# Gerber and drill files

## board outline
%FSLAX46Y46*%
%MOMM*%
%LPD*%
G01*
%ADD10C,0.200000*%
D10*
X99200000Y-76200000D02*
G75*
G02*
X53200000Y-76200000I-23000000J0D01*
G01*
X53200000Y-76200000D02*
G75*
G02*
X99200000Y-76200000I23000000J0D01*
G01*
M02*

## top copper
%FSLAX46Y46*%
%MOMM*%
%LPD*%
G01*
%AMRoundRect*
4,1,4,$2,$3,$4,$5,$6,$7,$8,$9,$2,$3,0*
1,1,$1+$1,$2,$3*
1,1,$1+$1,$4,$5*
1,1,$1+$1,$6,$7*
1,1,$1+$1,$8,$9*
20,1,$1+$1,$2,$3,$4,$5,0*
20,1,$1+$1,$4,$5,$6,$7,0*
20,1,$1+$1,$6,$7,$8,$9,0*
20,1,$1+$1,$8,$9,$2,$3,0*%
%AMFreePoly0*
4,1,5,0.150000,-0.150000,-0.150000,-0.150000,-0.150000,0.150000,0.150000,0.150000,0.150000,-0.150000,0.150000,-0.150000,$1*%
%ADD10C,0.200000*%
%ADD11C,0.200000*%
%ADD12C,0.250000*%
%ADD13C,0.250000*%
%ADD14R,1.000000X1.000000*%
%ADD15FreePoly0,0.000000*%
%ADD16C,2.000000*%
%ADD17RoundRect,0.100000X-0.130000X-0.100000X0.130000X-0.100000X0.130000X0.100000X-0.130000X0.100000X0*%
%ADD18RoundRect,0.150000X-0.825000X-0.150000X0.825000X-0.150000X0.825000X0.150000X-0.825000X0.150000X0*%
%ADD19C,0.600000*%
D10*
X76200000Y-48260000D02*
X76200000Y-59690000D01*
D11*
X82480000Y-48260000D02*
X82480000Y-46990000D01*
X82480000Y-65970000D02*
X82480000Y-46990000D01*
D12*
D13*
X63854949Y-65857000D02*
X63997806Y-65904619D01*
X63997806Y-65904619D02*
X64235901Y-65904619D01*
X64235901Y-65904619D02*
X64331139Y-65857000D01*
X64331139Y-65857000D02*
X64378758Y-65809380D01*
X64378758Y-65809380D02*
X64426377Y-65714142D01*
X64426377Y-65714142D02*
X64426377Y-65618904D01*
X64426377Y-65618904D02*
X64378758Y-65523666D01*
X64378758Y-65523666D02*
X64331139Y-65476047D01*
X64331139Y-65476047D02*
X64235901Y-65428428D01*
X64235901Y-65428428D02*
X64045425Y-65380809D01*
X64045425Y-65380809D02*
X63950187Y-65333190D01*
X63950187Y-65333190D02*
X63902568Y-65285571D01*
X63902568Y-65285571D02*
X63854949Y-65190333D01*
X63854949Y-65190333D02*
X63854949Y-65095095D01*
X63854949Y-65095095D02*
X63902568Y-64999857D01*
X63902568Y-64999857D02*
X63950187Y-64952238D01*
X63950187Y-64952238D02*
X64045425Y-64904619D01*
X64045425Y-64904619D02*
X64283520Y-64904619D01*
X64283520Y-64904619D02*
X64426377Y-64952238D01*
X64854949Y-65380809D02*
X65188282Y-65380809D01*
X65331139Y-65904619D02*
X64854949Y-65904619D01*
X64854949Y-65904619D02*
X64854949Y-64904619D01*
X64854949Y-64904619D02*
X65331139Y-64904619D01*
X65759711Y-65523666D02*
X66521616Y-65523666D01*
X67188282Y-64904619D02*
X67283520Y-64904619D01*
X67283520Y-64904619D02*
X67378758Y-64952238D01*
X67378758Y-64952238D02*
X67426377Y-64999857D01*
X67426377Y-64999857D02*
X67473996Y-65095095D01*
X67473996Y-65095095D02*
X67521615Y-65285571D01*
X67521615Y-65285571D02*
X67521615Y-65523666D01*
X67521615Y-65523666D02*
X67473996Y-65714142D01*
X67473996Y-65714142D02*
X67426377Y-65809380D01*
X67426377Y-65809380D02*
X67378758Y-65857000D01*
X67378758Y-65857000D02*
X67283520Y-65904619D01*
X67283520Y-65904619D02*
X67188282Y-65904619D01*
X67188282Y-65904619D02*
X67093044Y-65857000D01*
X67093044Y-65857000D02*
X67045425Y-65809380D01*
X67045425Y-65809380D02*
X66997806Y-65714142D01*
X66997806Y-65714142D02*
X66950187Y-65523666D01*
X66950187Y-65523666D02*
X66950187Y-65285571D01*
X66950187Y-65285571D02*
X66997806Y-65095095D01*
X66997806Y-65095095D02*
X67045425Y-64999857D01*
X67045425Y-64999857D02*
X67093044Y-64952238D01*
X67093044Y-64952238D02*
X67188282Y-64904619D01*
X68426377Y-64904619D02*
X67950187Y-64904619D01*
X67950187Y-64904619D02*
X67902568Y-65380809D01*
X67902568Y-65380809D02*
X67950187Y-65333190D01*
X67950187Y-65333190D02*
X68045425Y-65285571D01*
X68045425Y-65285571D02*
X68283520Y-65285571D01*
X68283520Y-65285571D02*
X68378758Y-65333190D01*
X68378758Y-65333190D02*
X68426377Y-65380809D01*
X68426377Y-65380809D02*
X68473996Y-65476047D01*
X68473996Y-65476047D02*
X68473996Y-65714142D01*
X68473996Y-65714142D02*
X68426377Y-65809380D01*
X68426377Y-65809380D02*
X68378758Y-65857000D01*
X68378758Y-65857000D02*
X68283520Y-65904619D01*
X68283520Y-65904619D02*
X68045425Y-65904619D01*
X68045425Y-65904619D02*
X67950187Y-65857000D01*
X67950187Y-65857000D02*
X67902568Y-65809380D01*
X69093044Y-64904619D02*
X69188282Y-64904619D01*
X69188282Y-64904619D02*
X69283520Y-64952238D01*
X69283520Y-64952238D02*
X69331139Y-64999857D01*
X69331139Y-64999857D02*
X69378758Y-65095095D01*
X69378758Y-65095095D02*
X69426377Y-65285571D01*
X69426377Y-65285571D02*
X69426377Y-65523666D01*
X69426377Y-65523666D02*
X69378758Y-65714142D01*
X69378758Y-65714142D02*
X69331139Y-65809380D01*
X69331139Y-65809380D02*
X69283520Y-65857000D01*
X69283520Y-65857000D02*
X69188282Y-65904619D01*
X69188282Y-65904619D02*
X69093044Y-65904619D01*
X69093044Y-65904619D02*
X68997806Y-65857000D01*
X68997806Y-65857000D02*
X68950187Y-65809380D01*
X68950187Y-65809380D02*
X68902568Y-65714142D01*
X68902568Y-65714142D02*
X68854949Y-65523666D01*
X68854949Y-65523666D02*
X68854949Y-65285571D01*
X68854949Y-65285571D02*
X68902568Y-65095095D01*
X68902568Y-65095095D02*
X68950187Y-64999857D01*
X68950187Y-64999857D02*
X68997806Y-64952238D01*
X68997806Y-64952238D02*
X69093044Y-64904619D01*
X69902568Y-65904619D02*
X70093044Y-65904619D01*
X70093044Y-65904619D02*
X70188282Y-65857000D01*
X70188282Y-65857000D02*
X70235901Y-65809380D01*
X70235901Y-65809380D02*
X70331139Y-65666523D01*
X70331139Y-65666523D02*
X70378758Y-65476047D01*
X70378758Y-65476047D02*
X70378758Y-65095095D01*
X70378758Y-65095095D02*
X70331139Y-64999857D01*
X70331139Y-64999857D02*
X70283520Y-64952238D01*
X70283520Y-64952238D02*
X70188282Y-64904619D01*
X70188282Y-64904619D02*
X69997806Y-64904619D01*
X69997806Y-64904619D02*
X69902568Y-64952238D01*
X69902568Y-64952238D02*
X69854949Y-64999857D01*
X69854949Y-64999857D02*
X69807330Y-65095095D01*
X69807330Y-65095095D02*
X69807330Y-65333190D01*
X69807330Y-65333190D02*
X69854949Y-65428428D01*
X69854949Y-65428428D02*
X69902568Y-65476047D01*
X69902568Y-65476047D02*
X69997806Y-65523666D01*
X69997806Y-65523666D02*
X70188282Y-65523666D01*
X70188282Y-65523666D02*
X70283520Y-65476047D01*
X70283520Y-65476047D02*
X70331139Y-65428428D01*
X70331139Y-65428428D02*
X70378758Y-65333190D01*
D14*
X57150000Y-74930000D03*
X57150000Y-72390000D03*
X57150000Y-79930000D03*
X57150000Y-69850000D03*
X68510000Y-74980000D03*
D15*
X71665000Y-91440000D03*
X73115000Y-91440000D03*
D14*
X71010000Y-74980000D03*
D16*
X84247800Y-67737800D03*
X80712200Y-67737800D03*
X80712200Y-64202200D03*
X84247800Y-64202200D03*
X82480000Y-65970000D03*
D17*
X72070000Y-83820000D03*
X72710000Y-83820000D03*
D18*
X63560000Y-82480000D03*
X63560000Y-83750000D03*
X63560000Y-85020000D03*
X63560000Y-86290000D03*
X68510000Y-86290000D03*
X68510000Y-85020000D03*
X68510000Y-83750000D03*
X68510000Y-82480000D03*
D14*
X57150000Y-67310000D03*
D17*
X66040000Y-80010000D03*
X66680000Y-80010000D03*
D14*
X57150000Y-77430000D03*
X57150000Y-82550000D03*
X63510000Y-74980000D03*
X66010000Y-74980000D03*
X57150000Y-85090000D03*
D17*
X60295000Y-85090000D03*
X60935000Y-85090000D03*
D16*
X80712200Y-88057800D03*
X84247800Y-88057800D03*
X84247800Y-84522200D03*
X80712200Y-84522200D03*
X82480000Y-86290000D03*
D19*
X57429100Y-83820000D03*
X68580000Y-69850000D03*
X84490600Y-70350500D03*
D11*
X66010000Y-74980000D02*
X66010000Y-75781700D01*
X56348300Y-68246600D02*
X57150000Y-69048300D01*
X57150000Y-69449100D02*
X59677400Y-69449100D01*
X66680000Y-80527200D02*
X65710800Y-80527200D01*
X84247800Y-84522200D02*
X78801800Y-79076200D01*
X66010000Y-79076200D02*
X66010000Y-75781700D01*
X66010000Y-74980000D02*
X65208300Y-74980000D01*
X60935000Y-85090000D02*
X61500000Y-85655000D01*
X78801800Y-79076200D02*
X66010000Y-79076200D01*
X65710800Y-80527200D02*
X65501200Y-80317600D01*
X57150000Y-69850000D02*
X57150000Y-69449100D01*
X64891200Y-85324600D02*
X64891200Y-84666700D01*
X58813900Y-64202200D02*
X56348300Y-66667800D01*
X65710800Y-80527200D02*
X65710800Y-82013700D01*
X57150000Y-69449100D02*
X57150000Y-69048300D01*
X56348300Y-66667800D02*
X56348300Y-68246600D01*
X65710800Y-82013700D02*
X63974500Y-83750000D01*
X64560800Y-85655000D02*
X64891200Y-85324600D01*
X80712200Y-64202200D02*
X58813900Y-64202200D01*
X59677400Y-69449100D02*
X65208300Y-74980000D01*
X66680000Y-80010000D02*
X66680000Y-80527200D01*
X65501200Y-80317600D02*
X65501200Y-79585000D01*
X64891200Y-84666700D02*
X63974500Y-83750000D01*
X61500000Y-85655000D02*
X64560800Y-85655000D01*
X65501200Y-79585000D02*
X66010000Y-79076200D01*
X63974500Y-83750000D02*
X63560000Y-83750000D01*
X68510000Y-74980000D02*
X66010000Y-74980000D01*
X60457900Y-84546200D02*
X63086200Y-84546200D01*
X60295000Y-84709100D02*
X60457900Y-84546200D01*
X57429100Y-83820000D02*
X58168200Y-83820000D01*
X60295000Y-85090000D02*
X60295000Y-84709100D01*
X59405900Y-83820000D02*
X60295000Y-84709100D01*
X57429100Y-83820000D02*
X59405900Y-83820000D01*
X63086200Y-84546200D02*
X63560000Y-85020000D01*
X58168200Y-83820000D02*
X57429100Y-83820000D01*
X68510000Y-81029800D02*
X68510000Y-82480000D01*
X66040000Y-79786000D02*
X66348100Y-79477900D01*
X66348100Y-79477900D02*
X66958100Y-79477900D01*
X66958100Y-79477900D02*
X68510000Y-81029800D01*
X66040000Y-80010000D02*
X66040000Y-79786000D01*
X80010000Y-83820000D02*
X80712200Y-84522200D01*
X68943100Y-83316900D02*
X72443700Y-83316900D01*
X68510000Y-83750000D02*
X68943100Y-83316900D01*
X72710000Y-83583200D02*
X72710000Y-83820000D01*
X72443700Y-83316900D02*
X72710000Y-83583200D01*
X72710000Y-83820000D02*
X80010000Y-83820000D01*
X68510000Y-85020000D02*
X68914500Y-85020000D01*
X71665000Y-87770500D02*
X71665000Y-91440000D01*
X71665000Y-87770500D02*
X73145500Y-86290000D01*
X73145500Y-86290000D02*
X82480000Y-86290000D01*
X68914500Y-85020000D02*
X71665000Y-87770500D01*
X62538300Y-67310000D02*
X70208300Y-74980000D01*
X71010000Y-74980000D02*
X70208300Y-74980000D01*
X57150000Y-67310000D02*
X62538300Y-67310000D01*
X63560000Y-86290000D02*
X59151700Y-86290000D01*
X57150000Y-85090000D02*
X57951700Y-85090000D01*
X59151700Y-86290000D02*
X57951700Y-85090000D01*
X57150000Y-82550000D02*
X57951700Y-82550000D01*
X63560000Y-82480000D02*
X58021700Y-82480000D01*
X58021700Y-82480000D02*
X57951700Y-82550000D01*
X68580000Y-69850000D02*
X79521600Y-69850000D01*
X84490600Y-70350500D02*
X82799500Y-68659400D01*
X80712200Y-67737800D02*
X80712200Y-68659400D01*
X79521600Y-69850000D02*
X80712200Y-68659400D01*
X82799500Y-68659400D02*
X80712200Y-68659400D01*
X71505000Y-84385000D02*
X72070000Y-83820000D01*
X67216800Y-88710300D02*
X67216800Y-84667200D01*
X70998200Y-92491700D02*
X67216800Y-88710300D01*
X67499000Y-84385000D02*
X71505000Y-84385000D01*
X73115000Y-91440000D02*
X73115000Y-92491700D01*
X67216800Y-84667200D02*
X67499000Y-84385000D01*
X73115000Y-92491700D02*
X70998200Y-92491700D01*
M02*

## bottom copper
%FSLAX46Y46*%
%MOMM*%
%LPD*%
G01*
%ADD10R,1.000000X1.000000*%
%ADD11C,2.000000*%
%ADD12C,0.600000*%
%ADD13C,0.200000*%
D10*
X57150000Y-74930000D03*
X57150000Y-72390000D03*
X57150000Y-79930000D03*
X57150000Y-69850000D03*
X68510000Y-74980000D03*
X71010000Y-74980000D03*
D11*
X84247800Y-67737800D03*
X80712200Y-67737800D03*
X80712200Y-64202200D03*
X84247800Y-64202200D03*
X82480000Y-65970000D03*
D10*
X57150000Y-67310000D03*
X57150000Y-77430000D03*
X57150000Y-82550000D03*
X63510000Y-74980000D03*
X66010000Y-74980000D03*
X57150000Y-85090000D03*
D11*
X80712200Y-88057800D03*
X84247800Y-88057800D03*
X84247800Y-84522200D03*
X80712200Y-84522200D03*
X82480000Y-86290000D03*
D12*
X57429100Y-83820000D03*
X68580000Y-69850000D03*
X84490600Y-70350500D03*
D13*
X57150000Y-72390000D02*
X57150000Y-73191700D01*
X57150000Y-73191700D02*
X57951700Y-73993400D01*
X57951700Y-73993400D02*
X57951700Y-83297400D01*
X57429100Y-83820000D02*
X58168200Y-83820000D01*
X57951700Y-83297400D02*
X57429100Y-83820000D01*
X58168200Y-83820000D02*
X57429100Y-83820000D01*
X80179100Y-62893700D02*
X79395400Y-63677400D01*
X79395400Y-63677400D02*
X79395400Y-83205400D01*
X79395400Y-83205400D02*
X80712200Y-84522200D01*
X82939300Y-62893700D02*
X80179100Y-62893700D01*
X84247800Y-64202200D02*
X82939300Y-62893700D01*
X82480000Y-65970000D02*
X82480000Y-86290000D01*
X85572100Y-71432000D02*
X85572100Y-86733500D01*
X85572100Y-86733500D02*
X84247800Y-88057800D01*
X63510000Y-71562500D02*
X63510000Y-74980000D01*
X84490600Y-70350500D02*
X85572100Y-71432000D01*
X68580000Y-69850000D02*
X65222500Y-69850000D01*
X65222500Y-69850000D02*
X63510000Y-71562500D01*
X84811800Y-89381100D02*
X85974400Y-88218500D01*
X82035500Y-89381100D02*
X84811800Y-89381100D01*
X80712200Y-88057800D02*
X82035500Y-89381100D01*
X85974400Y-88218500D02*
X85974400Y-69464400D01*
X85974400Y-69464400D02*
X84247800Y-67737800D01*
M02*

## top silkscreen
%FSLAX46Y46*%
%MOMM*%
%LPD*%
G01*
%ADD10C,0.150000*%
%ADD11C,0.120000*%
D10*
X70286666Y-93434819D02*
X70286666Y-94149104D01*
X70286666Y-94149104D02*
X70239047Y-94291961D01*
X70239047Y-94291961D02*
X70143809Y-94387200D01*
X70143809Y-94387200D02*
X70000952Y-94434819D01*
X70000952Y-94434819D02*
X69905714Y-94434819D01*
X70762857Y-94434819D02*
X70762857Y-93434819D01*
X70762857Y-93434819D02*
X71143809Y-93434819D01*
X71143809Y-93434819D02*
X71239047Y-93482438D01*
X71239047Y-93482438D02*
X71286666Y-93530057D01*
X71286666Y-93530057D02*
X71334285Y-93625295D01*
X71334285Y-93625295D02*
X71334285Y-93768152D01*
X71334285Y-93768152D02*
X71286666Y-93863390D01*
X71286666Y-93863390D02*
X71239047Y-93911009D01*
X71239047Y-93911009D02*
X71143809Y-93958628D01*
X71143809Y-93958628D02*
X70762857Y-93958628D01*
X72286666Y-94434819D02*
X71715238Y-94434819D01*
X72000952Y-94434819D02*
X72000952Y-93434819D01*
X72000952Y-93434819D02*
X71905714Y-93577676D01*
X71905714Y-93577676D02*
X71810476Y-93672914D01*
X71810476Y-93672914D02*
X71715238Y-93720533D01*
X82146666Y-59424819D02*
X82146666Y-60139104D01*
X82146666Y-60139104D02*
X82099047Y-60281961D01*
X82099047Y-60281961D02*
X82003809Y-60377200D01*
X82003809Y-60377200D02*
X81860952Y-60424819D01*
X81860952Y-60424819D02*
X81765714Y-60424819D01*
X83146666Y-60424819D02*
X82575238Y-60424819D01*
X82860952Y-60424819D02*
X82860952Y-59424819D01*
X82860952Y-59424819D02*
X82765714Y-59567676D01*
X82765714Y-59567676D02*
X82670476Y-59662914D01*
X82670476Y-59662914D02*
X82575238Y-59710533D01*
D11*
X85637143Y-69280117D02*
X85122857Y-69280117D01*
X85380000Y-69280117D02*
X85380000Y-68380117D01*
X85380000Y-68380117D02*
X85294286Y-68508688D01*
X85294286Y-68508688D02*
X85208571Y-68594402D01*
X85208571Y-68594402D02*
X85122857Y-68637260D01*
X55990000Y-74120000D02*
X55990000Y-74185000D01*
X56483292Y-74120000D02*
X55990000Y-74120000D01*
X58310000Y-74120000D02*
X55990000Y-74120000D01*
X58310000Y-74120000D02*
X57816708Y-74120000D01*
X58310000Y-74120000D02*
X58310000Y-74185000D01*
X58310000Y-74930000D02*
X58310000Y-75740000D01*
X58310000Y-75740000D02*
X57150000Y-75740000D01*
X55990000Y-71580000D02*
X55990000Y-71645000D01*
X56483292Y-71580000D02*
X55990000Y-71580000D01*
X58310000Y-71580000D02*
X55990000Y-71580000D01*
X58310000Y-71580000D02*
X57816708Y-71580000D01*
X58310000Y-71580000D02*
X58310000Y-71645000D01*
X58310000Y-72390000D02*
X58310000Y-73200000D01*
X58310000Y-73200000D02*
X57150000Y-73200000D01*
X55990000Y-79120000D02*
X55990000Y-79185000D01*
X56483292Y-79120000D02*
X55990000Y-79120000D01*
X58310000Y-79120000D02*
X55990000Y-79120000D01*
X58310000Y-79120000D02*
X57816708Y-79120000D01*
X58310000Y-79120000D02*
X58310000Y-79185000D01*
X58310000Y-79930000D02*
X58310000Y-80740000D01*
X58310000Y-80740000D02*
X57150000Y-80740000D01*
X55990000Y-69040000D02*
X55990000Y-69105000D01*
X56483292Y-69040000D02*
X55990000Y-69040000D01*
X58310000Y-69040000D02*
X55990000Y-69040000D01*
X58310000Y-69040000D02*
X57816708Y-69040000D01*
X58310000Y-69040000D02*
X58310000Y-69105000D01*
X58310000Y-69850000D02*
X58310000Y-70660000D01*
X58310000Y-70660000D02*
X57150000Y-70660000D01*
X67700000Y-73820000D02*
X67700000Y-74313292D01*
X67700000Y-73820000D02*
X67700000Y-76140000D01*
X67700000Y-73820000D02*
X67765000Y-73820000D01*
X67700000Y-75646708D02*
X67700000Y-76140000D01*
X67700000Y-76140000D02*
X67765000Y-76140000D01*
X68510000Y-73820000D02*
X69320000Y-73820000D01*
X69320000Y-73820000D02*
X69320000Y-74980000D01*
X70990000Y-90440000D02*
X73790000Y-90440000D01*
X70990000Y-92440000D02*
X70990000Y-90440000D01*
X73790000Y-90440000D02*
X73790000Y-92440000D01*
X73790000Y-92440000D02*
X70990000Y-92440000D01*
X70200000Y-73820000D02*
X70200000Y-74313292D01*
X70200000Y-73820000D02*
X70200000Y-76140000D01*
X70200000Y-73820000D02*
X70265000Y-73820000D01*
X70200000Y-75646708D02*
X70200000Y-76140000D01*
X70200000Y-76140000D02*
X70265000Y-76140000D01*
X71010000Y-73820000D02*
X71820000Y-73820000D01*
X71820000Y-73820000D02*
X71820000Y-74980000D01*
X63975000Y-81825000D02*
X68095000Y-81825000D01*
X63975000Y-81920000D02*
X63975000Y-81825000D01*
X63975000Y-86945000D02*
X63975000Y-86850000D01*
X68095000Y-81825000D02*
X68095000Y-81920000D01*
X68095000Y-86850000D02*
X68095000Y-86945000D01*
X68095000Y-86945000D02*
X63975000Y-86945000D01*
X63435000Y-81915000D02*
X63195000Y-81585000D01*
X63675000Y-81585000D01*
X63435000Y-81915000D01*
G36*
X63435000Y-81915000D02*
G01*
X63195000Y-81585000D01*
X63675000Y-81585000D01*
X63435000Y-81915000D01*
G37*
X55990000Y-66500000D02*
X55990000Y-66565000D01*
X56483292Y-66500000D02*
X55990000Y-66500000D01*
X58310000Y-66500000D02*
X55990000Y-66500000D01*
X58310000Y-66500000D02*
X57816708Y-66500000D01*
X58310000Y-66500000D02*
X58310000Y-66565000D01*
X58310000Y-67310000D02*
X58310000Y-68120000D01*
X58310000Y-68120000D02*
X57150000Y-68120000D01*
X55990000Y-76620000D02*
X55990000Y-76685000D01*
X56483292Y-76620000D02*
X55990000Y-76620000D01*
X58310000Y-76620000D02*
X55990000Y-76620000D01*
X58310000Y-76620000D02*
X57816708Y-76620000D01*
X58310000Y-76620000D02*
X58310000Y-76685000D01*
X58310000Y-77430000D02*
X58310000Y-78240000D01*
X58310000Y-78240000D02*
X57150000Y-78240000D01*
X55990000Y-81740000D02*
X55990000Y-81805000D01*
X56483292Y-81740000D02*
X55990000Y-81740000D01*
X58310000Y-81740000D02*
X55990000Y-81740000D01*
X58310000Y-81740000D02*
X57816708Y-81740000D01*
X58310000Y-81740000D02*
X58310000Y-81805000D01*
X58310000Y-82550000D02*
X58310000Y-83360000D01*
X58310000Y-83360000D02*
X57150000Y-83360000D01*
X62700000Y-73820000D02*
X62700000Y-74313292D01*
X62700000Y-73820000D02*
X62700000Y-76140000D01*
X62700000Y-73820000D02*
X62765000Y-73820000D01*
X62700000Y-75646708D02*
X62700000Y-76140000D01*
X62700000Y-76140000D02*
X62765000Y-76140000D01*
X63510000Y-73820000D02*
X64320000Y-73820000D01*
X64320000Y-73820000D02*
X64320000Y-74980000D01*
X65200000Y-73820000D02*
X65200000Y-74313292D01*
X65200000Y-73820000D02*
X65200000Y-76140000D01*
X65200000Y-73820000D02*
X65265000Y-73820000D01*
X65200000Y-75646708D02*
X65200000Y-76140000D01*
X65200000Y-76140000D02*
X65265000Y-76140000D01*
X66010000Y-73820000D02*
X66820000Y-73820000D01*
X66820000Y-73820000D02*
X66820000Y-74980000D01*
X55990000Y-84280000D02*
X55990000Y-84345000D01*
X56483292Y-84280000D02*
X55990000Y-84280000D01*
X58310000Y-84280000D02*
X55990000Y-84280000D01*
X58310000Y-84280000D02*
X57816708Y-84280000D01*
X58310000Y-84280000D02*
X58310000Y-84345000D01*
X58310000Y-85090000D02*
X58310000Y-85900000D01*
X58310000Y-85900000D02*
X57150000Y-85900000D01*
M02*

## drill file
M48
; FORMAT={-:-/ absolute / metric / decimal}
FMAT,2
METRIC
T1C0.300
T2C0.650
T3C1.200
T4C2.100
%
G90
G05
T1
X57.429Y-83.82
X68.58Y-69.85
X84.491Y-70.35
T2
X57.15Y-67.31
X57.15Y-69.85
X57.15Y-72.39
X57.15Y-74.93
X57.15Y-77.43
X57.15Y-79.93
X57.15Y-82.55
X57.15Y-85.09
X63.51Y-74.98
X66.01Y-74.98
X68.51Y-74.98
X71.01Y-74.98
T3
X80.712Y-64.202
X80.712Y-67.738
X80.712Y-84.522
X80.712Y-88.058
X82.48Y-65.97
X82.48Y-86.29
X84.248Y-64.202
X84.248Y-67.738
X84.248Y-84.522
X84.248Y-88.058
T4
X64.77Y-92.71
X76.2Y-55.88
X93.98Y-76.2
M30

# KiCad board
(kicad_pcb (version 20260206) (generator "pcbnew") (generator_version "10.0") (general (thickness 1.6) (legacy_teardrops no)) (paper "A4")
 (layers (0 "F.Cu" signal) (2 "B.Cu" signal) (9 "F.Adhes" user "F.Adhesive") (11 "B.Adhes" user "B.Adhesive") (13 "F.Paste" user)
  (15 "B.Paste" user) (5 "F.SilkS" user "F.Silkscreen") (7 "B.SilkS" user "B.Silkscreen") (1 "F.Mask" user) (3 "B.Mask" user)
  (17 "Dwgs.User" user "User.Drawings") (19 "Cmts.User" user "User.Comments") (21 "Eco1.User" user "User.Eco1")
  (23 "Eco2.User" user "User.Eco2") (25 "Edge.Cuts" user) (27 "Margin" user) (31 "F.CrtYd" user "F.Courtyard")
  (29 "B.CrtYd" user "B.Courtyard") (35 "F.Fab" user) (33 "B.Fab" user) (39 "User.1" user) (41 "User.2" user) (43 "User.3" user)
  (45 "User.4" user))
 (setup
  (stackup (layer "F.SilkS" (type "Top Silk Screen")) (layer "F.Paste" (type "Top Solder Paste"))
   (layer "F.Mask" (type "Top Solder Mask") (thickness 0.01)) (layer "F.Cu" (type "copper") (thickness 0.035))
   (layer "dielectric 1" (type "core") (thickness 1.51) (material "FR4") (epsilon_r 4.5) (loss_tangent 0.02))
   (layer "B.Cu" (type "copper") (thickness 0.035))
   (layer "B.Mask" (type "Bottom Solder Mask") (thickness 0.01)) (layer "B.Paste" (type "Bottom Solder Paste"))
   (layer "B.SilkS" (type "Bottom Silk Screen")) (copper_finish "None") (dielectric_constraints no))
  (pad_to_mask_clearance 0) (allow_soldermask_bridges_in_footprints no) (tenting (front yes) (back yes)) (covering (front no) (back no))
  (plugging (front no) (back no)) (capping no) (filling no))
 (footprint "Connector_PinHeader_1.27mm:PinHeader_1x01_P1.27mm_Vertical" (layer "F.Cu") (at 57.15 74.93 180)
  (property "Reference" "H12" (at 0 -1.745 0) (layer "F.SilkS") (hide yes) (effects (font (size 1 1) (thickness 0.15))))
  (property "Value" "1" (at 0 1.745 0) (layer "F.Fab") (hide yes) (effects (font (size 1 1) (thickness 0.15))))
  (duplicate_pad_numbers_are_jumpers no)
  (fp_line (start 1.16 0.81) (end 1.16 0.745) (stroke (width 0.12) (type solid)) (layer "F.SilkS"))
  (fp_line (start 0.666708 0.81) (end 1.16 0.81) (stroke (width 0.12) (type solid)) (layer "F.SilkS"))
  (fp_line (start -1.16 0.81) (end 1.16 0.81) (stroke (width 0.12) (type solid)) (layer "F.SilkS"))
  (fp_line (start -1.16 0.81) (end -0.666708 0.81) (stroke (width 0.12) (type solid)) (layer "F.SilkS"))
  (fp_line (start -1.16 0.81) (end -1.16 0.745) (stroke (width 0.12) (type solid)) (layer "F.SilkS"))
  (fp_line (start -1.16 0) (end -1.16 -0.81) (stroke (width 0.12) (type solid)) (layer "F.SilkS"))
  (fp_line (start -1.16 -0.81) (end 0 -0.81) (stroke (width 0.12) (type solid)) (layer "F.SilkS"))
  (pad "1" thru_hole rect (at 0 0 180) (size 1 1) (drill 0.65) (layers "*.Cu" "*.Mask") (remove_unused_layers no)
   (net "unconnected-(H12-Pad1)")))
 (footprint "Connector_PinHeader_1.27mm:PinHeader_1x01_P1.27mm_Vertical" (layer "F.Cu") (at 57.15 72.39 180)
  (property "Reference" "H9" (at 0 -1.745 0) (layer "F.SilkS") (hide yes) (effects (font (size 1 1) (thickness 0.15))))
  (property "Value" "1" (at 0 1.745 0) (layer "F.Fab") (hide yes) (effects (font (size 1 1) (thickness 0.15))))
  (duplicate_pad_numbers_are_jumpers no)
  (fp_line (start 1.16 0.81) (end 1.16 0.745) (stroke (width 0.12) (type solid)) (layer "F.SilkS"))
  (fp_line (start 0.666708 0.81) (end 1.16 0.81) (stroke (width 0.12) (type solid)) (layer "F.SilkS"))
  (fp_line (start -1.16 0.81) (end 1.16 0.81) (stroke (width 0.12) (type solid)) (layer "F.SilkS"))
  (fp_line (start -1.16 0.81) (end -0.666708 0.81) (stroke (width 0.12) (type solid)) (layer "F.SilkS"))
  (fp_line (start -1.16 0.81) (end -1.16 0.745) (stroke (width 0.12) (type solid)) (layer "F.SilkS"))
  (fp_line (start -1.16 0) (end -1.16 -0.81) (stroke (width 0.12) (type solid)) (layer "F.SilkS"))
  (fp_line (start -1.16 -0.81) (end 0 -0.81) (stroke (width 0.12) (type solid)) (layer "F.SilkS"))
  (pad "1" thru_hole rect (at 0 0 180) (size 1 1) (drill 0.65) (layers "*.Cu" "*.Mask") (remove_unused_layers no) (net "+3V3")))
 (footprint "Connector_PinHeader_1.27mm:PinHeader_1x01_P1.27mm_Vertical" (layer "F.Cu") (at 57.15 79.93 180)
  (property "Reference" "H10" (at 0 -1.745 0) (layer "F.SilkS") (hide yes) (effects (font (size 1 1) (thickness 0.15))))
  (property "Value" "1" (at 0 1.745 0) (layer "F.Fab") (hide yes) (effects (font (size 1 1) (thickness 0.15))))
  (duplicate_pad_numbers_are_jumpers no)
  (fp_line (start 1.16 0.81) (end 1.16 0.745) (stroke (width 0.12) (type solid)) (layer "F.SilkS"))
  (fp_line (start 0.666708 0.81) (end 1.16 0.81) (stroke (width 0.12) (type solid)) (layer "F.SilkS"))
  (fp_line (start -1.16 0.81) (end 1.16 0.81) (stroke (width 0.12) (type solid)) (layer "F.SilkS"))
  (fp_line (start -1.16 0.81) (end -0.666708 0.81) (stroke (width 0.12) (type solid)) (layer "F.SilkS"))
  (fp_line (start -1.16 0.81) (end -1.16 0.745) (stroke (width 0.12) (type solid)) (layer "F.SilkS"))
  (fp_line (start -1.16 0) (end -1.16 -0.81) (stroke (width 0.12) (type solid)) (layer "F.SilkS"))
  (fp_line (start -1.16 -0.81) (end 0 -0.81) (stroke (width 0.12) (type solid)) (layer "F.SilkS"))
  (pad "1" thru_hole rect (at 0 0 180) (size 1 1) (drill 0.65) (layers "*.Cu" "*.Mask") (remove_unused_layers no)
   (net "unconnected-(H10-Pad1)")))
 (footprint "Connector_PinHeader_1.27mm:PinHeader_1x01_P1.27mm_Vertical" (layer "F.Cu") (at 57.15 69.85 180)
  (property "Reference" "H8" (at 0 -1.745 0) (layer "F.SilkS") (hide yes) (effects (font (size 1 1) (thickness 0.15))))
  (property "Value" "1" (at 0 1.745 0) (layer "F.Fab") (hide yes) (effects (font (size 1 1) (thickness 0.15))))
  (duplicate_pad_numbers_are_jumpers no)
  (fp_line (start 1.16 0.81) (end 1.16 0.745) (stroke (width 0.12) (type solid)) (layer "F.SilkS"))
  (fp_line (start 0.666708 0.81) (end 1.16 0.81) (stroke (width 0.12) (type solid)) (layer "F.SilkS"))
  (fp_line (start -1.16 0.81) (end 1.16 0.81) (stroke (width 0.12) (type solid)) (layer "F.SilkS"))
  (fp_line (start -1.16 0.81) (end -0.666708 0.81) (stroke (width 0.12) (type solid)) (layer "F.SilkS"))
  (fp_line (start -1.16 0.81) (end -1.16 0.745) (stroke (width 0.12) (type solid)) (layer "F.SilkS"))
  (fp_line (start -1.16 0) (end -1.16 -0.81) (stroke (width 0.12) (type solid)) (layer "F.SilkS"))
  (fp_line (start -1.16 -0.81) (end 0 -0.81) (stroke (width 0.12) (type solid)) (layer "F.SilkS"))
  (pad "1" thru_hole rect (at 0 0 180) (size 1 1) (drill 0.65) (layers "*.Cu" "*.Mask") (remove_unused_layers no) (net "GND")))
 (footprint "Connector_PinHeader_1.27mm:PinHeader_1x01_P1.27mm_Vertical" (layer "F.Cu") (at 68.51 74.98 -90)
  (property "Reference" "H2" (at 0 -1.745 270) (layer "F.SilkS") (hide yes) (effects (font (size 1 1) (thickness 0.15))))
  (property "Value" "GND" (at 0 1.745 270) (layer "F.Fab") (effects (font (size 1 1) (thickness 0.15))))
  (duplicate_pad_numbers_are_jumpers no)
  (fp_line (start -1.16 0.81) (end -0.666708 0.81) (stroke (width 0.12) (type solid)) (layer "F.SilkS"))
  (fp_line (start -1.16 0.81) (end 1.16 0.81) (stroke (width 0.12) (type solid)) (layer "F.SilkS"))
  (fp_line (start -1.16 0.81) (end -1.16 0.745) (stroke (width 0.12) (type solid)) (layer "F.SilkS"))
  (fp_line (start 0.666708 0.81) (end 1.16 0.81) (stroke (width 0.12) (type solid)) (layer "F.SilkS"))
  (fp_line (start 1.16 0.81) (end 1.16 0.745) (stroke (width 0.12) (type solid)) (layer "F.SilkS"))
  (fp_line (start -1.16 0) (end -1.16 -0.81) (stroke (width 0.12) (type solid)) (layer "F.SilkS"))
  (fp_line (start -1.16 -0.81) (end 0 -0.81) (stroke (width 0.12) (type solid)) (layer "F.SilkS"))
  (pad "1" thru_hole rect (at 0 0 270) (size 1 1) (drill 0.65) (layers "*.Cu" "*.Mask") (remove_unused_layers no) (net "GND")))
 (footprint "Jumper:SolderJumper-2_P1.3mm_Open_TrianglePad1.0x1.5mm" (layer "F.Cu") (at 72.39 91.44)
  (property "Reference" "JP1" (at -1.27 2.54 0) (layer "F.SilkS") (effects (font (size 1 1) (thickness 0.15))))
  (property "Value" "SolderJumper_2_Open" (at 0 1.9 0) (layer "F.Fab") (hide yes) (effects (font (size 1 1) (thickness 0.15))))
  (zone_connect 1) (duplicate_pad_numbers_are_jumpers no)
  (fp_line (start -1.4 -1) (end 1.4 -1) (stroke (width 0.12) (type solid)) (layer "F.SilkS"))
  (fp_line (start -1.4 1) (end -1.4 -1) (stroke (width 0.12) (type solid)) (layer "F.SilkS"))
  (fp_line (start 1.4 -1) (end 1.4 1) (stroke (width 0.12) (type solid)) (layer "F.SilkS"))
  (fp_line (start 1.4 1) (end -1.4 1) (stroke (width 0.12) (type solid)) (layer "F.SilkS"))
  (pad "1" smd custom (at -0.725 0) (size 0.3 0.3) (layers "F.Cu" "F.Mask") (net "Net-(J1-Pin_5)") (zone_connect 2)
   (thermal_bridge_angle 45) (options (clearance outline) (anchor rect)) (primitives))
  (pad "2" smd custom (at 0.725 0) (size 0.3 0.3) (layers "F.Cu" "F.Mask") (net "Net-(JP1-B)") (zone_connect 2) (thermal_bridge_angle 45)
   (options (clearance outline) (anchor rect)) (primitives)))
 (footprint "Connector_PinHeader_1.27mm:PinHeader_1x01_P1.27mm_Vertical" (layer "F.Cu") (at 71.01 74.98 -90)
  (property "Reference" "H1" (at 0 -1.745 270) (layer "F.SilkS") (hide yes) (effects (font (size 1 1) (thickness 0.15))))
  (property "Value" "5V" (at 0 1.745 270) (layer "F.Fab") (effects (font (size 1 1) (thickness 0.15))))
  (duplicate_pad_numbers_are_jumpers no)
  (fp_line (start -1.16 0.81) (end -0.666708 0.81) (stroke (width 0.12) (type solid)) (layer "F.SilkS"))
  (fp_line (start -1.16 0.81) (end 1.16 0.81) (stroke (width 0.12) (type solid)) (layer "F.SilkS"))
  (fp_line (start -1.16 0.81) (end -1.16 0.745) (stroke (width 0.12) (type solid)) (layer "F.SilkS"))
  (fp_line (start 0.666708 0.81) (end 1.16 0.81) (stroke (width 0.12) (type solid)) (layer "F.SilkS"))
  (fp_line (start 1.16 0.81) (end 1.16 0.745) (stroke (width 0.12) (type solid)) (layer "F.SilkS"))
  (fp_line (start -1.16 0) (end -1.16 -0.81) (stroke (width 0.12) (type solid)) (layer "F.SilkS"))
  (fp_line (start -1.16 -0.81) (end 0 -0.81) (stroke (width 0.12) (type solid)) (layer "F.SilkS"))
  (pad "1" thru_hole rect (at 0 0 270) (size 1 1) (drill 0.65) (layers "*.Cu" "*.Mask") (remove_unused_layers no) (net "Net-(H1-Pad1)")))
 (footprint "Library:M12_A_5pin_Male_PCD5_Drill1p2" (layer "F.Cu") (at 82.48 65.97)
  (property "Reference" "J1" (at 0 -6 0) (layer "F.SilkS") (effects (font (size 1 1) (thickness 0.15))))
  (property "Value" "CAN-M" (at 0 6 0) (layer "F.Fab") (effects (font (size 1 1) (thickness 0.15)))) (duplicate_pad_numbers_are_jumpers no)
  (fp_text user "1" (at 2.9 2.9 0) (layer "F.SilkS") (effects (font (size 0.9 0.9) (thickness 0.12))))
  (pad "1" thru_hole circle (at 1.7678 1.7678) (size 2 2) (drill 1.2) (layers "*.Cu" "*.Mask") (remove_unused_layers no)
   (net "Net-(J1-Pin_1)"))
  (pad "2" thru_hole circle (at -1.7678 1.7678) (size 2 2) (drill 1.2) (layers "*.Cu" "*.Mask") (remove_unused_layers no) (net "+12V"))
  (pad "3" thru_hole circle (at -1.7678 -1.7678) (size 2 2) (drill 1.2) (layers "*.Cu" "*.Mask") (remove_unused_layers no) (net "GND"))
  (pad "4" thru_hole circle (at 1.7678 -1.7678) (size 2 2) (drill 1.2) (layers "*.Cu" "*.Mask") (remove_unused_layers no)
   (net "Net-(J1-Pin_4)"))
  (pad "5" thru_hole circle (at 0 0) (size 2 2) (drill 1.2) (layers "*.Cu" "*.Mask") (remove_unused_layers no) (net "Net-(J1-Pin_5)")))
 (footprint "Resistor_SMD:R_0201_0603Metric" (layer "F.Cu") (at 72.39 83.82)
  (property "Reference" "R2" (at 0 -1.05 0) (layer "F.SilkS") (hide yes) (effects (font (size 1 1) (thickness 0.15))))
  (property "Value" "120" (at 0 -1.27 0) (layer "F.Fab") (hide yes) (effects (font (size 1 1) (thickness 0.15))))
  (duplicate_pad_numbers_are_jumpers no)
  (pad "" smd roundrect (at -0.345 0) (size 0.318 0.36) (layers "F.Paste") (roundrect_rratio 0.25))
  (pad "" smd roundrect (at 0.345 0) (size 0.318 0.36) (layers "F.Paste") (roundrect_rratio 0.25))
  (pad "1" smd roundrect (at -0.32 0) (size 0.46 0.4) (layers "F.Cu" "F.Mask") (roundrect_rratio 0.25) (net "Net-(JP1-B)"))
  (pad "2" smd roundrect (at 0.32 0) (size 0.46 0.4) (layers "F.Cu" "F.Mask") (roundrect_rratio 0.25) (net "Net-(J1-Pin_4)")))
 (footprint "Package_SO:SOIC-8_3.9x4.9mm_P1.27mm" (layer "F.Cu") (at 66.035 84.385)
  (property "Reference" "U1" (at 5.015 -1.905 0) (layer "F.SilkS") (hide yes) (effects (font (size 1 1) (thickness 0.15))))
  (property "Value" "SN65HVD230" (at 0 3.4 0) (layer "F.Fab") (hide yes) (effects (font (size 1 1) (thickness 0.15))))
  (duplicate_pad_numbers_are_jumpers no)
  (fp_line (start -2.06 -2.56) (end 2.06 -2.56) (stroke (width 0.12) (type solid)) (layer "F.SilkS"))
  (fp_line (start -2.06 -2.465) (end -2.06 -2.56) (stroke (width 0.12) (type solid)) (layer "F.SilkS"))
  (fp_line (start -2.06 2.56) (end -2.06 2.465) (stroke (width 0.12) (type solid)) (layer "F.SilkS"))
  (fp_line (start 2.06 -2.56) (end 2.06 -2.465) (stroke (width 0.12) (type solid)) (layer "F.SilkS"))
  (fp_line (start 2.06 2.465) (end 2.06 2.56) (stroke (width 0.12) (type solid)) (layer "F.SilkS"))
  (fp_line (start 2.06 2.56) (end -2.06 2.56) (stroke (width 0.12) (type solid)) (layer "F.SilkS"))
  (fp_poly (pts (xy -2.6 -2.47) (xy -2.84 -2.8) (xy -2.36 -2.8)) (stroke (width 0.12) (type solid)) (fill yes) (layer "F.SilkS"))
  (pad "1" smd roundrect (at -2.475 -1.905) (size 1.95 0.6) (layers "F.Cu" "F.Mask" "F.Paste") (roundrect_rratio 0.25) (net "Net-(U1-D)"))
  (pad "2" smd roundrect (at -2.475 -0.635) (size 1.95 0.6) (layers "F.Cu" "F.Mask" "F.Paste") (roundrect_rratio 0.25) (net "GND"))
  (pad "3" smd roundrect (at -2.475 0.635) (size 1.95 0.6) (layers "F.Cu" "F.Mask" "F.Paste") (roundrect_rratio 0.25) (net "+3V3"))
  (pad "4" smd roundrect (at -2.475 1.905) (size 1.95 0.6) (layers "F.Cu" "F.Mask" "F.Paste") (roundrect_rratio 0.25) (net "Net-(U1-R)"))
  (pad "5" smd roundrect (at 2.475 1.905) (size 1.95 0.6) (layers "F.Cu" "F.Mask" "F.Paste") (roundrect_rratio 0.25)
   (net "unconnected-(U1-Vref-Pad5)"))
  (pad "6" smd roundrect (at 2.475 0.635) (size 1.95 0.6) (layers "F.Cu" "F.Mask" "F.Paste") (roundrect_rratio 0.25) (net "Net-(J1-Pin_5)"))
  (pad "7" smd roundrect (at 2.475 -0.635) (size 1.95 0.6) (layers "F.Cu" "F.Mask" "F.Paste") (roundrect_rratio 0.25) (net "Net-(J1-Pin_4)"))
  (pad "8" smd roundrect (at 2.475 -1.905) (size 1.95 0.6) (layers "F.Cu" "F.Mask" "F.Paste") (roundrect_rratio 0.25) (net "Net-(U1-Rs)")))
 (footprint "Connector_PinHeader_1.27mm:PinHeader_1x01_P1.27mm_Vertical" (layer "F.Cu") (at 57.15 67.31 180)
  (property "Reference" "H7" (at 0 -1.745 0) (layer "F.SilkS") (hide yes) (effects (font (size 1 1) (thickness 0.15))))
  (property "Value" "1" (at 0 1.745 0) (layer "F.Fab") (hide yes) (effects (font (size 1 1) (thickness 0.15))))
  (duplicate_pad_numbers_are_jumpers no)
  (fp_line (start 1.16 0.81) (end 1.16 0.745) (stroke (width 0.12) (type solid)) (layer "F.SilkS"))
  (fp_line (start 0.666708 0.81) (end 1.16 0.81) (stroke (width 0.12) (type solid)) (layer "F.SilkS"))
  (fp_line (start -1.16 0.81) (end 1.16 0.81) (stroke (width 0.12) (type solid)) (layer "F.SilkS"))
  (fp_line (start -1.16 0.81) (end -0.666708 0.81) (stroke (width 0.12) (type solid)) (layer "F.SilkS"))
  (fp_line (start -1.16 0.81) (end -1.16 0.745) (stroke (width 0.12) (type solid)) (layer "F.SilkS"))
  (fp_line (start -1.16 0) (end -1.16 -0.81) (stroke (width 0.12) (type solid)) (layer "F.SilkS"))
  (fp_line (start -1.16 -0.81) (end 0 -0.81) (stroke (width 0.12) (type solid)) (layer "F.SilkS"))
  (pad "1" thru_hole rect (at 0 0 180) (size 1 1) (drill 0.65) (layers "*.Cu" "*.Mask") (remove_unused_layers no) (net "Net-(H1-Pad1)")))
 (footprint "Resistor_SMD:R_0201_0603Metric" (layer "F.Cu") (at 66.36 80.01)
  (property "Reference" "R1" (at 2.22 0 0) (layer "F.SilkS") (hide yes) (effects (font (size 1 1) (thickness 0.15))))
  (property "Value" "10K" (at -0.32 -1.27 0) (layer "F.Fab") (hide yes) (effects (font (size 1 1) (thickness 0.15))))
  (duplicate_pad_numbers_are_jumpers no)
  (pad "" smd roundrect (at -0.345 0) (size 0.318 0.36) (layers "F.Paste") (roundrect_rratio 0.25))
  (pad "" smd roundrect (at 0.345 0) (size 0.318 0.36) (layers "F.Paste") (roundrect_rratio 0.25))
  (pad "1" smd roundrect (at -0.32 0) (size 0.46 0.4) (layers "F.Cu" "F.Mask") (roundrect_rratio 0.25) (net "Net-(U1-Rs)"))
  (pad "2" smd roundrect (at 0.32 0) (size 0.46 0.4) (layers "F.Cu" "F.Mask") (roundrect_rratio 0.25) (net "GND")))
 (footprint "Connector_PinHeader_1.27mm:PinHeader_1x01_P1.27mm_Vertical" (layer "F.Cu") (at 57.15 77.43 180)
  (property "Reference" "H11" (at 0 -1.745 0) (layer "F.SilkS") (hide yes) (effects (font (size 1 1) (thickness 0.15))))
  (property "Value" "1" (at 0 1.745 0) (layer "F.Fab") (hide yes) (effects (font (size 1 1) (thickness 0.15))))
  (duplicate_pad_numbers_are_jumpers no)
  (fp_line (start 1.16 0.81) (end 1.16 0.745) (stroke (width 0.12) (type solid)) (layer "F.SilkS"))
  (fp_line (start 0.666708 0.81) (end 1.16 0.81) (stroke (width 0.12) (type solid)) (layer "F.SilkS"))
  (fp_line (start -1.16 0.81) (end 1.16 0.81) (stroke (width 0.12) (type solid)) (layer "F.SilkS"))
  (fp_line (start -1.16 0.81) (end -0.666708 0.81) (stroke (width 0.12) (type solid)) (layer "F.SilkS"))
  (fp_line (start -1.16 0.81) (end -1.16 0.745) (stroke (width 0.12) (type solid)) (layer "F.SilkS"))
  (fp_line (start -1.16 0) (end -1.16 -0.81) (stroke (width 0.12) (type solid)) (layer "F.SilkS"))
  (fp_line (start -1.16 -0.81) (end 0 -0.81) (stroke (width 0.12) (type solid)) (layer "F.SilkS"))
  (pad "1" thru_hole rect (at 0 0 180) (size 1 1) (drill 0.65) (layers "*.Cu" "*.Mask") (remove_unused_layers no)
   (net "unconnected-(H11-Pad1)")))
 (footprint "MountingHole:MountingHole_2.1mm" (layer "F.Cu") (at 93.98 76.2)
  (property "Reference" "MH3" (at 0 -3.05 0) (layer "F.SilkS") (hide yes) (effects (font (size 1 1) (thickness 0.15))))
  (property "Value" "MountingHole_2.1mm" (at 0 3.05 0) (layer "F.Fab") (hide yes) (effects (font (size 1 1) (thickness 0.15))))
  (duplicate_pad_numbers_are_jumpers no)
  (pad "" np_thru_hole circle (at 0 0) (size 2.1 2.1) (drill 2.1) (layers "*.Cu" "*.Mask")))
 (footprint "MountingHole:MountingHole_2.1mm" (layer "F.Cu") (at 64.77 92.71)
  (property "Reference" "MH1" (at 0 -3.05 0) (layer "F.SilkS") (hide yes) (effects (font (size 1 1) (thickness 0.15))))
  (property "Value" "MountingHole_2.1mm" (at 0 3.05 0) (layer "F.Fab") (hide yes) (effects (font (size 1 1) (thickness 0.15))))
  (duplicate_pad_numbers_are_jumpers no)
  (pad "" np_thru_hole circle (at 0 0) (size 2.1 2.1) (drill 2.1) (layers "*.Cu" "*.Mask")))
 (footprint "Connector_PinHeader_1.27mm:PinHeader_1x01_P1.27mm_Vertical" (layer "F.Cu") (at 57.15 82.55 180)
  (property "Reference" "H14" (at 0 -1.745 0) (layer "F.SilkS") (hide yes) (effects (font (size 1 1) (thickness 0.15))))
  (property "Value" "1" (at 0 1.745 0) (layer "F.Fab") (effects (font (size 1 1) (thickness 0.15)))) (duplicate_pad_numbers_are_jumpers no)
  (fp_line (start 1.16 0.81) (end 1.16 0.745) (stroke (width 0.12) (type solid)) (layer "F.SilkS"))
  (fp_line (start 0.666708 0.81) (end 1.16 0.81) (stroke (width 0.12) (type solid)) (layer "F.SilkS"))
  (fp_line (start -1.16 0.81) (end 1.16 0.81) (stroke (width 0.12) (type solid)) (layer "F.SilkS"))
  (fp_line (start -1.16 0.81) (end -0.666708 0.81) (stroke (width 0.12) (type solid)) (layer "F.SilkS"))
  (fp_line (start -1.16 0.81) (end -1.16 0.745) (stroke (width 0.12) (type solid)) (layer "F.SilkS"))
  (fp_line (start -1.16 0) (end -1.16 -0.81) (stroke (width 0.12) (type solid)) (layer "F.SilkS"))
  (fp_line (start -1.16 -0.81) (end 0 -0.81) (stroke (width 0.12) (type solid)) (layer "F.SilkS"))
  (pad "1" thru_hole rect (at 0 0 180) (size 1 1) (drill 0.65) (layers "*.Cu" "*.Mask") (remove_unused_layers no) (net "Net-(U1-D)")))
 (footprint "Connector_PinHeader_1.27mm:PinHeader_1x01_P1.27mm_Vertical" (layer "F.Cu") (at 63.51 74.98 -90)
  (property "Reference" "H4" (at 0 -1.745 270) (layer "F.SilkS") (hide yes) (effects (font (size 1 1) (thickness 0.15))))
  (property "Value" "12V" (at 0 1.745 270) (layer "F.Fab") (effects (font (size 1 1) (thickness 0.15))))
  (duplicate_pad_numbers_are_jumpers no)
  (fp_line (start -1.16 0.81) (end -0.666708 0.81) (stroke (width 0.12) (type solid)) (layer "F.SilkS"))
  (fp_line (start -1.16 0.81) (end 1.16 0.81) (stroke (width 0.12) (type solid)) (layer "F.SilkS"))
  (fp_line (start -1.16 0.81) (end -1.16 0.745) (stroke (width 0.12) (type solid)) (layer "F.SilkS"))
  (fp_line (start 0.666708 0.81) (end 1.16 0.81) (stroke (width 0.12) (type solid)) (layer "F.SilkS"))
  (fp_line (start 1.16 0.81) (end 1.16 0.745) (stroke (width 0.12) (type solid)) (layer "F.SilkS"))
  (fp_line (start -1.16 0) (end -1.16 -0.81) (stroke (width 0.12) (type solid)) (layer "F.SilkS"))
  (fp_line (start -1.16 -0.81) (end 0 -0.81) (stroke (width 0.12) (type solid)) (layer "F.SilkS"))
  (pad "1" thru_hole rect (at 0 0 270) (size 1 1) (drill 0.65) (layers "*.Cu" "*.Mask") (remove_unused_layers no) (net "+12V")))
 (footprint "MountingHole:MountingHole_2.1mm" (layer "F.Cu") (at 76.2 55.88)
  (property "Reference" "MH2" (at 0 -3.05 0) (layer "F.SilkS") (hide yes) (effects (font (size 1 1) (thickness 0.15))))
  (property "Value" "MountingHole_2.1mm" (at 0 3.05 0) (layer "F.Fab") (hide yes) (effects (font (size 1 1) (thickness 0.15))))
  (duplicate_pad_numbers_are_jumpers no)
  (pad "" np_thru_hole circle (at 0 0) (size 2.1 2.1) (drill 2.1) (layers "*.Cu" "*.Mask")))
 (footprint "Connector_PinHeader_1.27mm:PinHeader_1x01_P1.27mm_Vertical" (layer "F.Cu") (at 66.01 74.98 -90)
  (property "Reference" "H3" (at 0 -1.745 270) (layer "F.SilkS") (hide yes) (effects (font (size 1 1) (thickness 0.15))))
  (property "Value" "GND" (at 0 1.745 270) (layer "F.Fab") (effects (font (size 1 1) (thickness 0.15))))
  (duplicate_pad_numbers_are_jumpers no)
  (fp_line (start -1.16 0.81) (end -0.666708 0.81) (stroke (width 0.12) (type solid)) (layer "F.SilkS"))
  (fp_line (start -1.16 0.81) (end 1.16 0.81) (stroke (width 0.12) (type solid)) (layer "F.SilkS"))
  (fp_line (start -1.16 0.81) (end -1.16 0.745) (stroke (width 0.12) (type solid)) (layer "F.SilkS"))
  (fp_line (start 0.666708 0.81) (end 1.16 0.81) (stroke (width 0.12) (type solid)) (layer "F.SilkS"))
  (fp_line (start 1.16 0.81) (end 1.16 0.745) (stroke (width 0.12) (type solid)) (layer "F.SilkS"))
  (fp_line (start -1.16 0) (end -1.16 -0.81) (stroke (width 0.12) (type solid)) (layer "F.SilkS"))
  (fp_line (start -1.16 -0.81) (end 0 -0.81) (stroke (width 0.12) (type solid)) (layer "F.SilkS"))
  (pad "1" thru_hole rect (at 0 0 270) (size 1 1) (drill 0.65) (layers "*.Cu" "*.Mask") (remove_unused_layers no) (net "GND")))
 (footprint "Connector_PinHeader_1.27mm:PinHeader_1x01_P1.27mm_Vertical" (layer "F.Cu") (at 57.15 85.09 180)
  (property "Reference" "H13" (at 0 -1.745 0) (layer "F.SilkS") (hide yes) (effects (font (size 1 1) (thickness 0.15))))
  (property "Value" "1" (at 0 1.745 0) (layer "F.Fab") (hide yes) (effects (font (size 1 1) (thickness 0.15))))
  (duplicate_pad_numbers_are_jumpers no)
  (fp_line (start 1.16 0.81) (end 1.16 0.745) (stroke (width 0.12) (type solid)) (layer "F.SilkS"))
  (fp_line (start 0.666708 0.81) (end 1.16 0.81) (stroke (width 0.12) (type solid)) (layer "F.SilkS"))
  (fp_line (start -1.16 0.81) (end 1.16 0.81) (stroke (width 0.12) (type solid)) (layer "F.SilkS"))
  (fp_line (start -1.16 0.81) (end -0.666708 0.81) (stroke (width 0.12) (type solid)) (layer "F.SilkS"))
  (fp_line (start -1.16 0.81) (end -1.16 0.745) (stroke (width 0.12) (type solid)) (layer "F.SilkS"))
  (fp_line (start -1.16 0) (end -1.16 -0.81) (stroke (width 0.12) (type solid)) (layer "F.SilkS"))
  (fp_line (start -1.16 -0.81) (end 0 -0.81) (stroke (width 0.12) (type solid)) (layer "F.SilkS"))
  (pad "1" thru_hole rect (at 0 0 180) (size 1 1) (drill 0.65) (layers "*.Cu" "*.Mask") (remove_unused_layers no) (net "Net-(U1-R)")))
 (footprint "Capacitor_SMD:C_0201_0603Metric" (layer "F.Cu") (at 60.615 85.09)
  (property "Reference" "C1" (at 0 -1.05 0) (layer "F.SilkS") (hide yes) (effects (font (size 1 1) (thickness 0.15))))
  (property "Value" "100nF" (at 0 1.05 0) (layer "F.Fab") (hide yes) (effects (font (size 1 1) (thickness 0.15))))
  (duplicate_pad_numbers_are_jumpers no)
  (pad "" smd roundrect (at -0.345 0) (size 0.318 0.36) (layers "F.Paste") (roundrect_rratio 0.25))
  (pad "" smd roundrect (at 0.345 0) (size 0.318 0.36) (layers "F.Paste") (roundrect_rratio 0.25))
  (pad "1" smd roundrect (at -0.32 0) (size 0.46 0.4) (layers "F.Cu" "F.Mask") (roundrect_rratio 0.25) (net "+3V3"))
  (pad "2" smd roundrect (at 0.32 0) (size 0.46 0.4) (layers "F.Cu" "F.Mask") (roundrect_rratio 0.25) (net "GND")))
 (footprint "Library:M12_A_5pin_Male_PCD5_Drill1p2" (layer "B.Cu") (at 82.48 86.29 180)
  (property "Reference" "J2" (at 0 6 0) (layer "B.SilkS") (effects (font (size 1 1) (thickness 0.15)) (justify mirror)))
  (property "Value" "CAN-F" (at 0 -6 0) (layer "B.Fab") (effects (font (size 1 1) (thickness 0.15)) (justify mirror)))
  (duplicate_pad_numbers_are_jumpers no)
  (pad "1" thru_hole circle (at 1.7678 -1.7678 180) (size 2 2) (drill 1.2) (layers "*.Cu" "*.Mask") (remove_unused_layers no)
   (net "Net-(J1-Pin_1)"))
  (pad "2" thru_hole circle (at -1.7678 -1.7678 180) (size 2 2) (drill 1.2) (layers "*.Cu" "*.Mask") (remove_unused_layers no) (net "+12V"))
  (pad "3" thru_hole circle (at -1.7678 1.7678 180) (size 2 2) (drill 1.2) (layers "*.Cu" "*.Mask") (remove_unused_layers no) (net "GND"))
  (pad "4" thru_hole circle (at 1.7678 1.7678 180) (size 2 2) (drill 1.2) (layers "*.Cu" "*.Mask") (remove_unused_layers no)
   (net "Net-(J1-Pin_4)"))
  (pad "5" thru_hole circle (at 0 0 180) (size 2 2) (drill 1.2) (layers "*.Cu" "*.Mask") (remove_unused_layers no) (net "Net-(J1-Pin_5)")))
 (gr_line (start 76.2 48.26) (end 76.2 59.69) (stroke (width 0.2) (type default)) (layer "F.Cu"))
 (gr_line (start 82.48 48.26) (end 82.48 46.99) (stroke (width 0.2) (type default)) (layer "F.Cu") (net "Net-(J1-Pin_5)"))
 (gr_line (start 82.48 65.97) (end 82.48 46.99) (stroke (width 0.2) (type default)) (layer "F.Cu") (net "Net-(J1-Pin_5)"))
 (gr_circle (center 76.2 76.2) (end 99.2 76.2) (stroke (width 0.2) (type solid)) (fill no) (layer "Edge.Cuts"))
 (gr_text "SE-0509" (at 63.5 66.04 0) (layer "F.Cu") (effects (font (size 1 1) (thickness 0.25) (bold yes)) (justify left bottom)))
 (segment (start 66.01 74.98) (end 66.01 75.7817) (width 0.2) (layer "F.Cu") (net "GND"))
 (segment (start 56.3483 68.2466) (end 57.15 69.0483) (width 0.2) (layer "F.Cu") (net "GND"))
 (segment (start 57.15 69.4491) (end 59.6774 69.4491) (width 0.2) (layer "F.Cu") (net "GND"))
 (segment (start 66.68 80.5272) (end 65.7108 80.5272) (width 0.2) (layer "F.Cu") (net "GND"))
 (segment (start 84.2478 84.5222) (end 78.8018 79.0762) (width 0.2) (layer "F.Cu") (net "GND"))
 (segment (start 66.01 79.0762) (end 66.01 75.7817) (width 0.2) (layer "F.Cu") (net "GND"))
 (segment (start 66.01 74.98) (end 65.2083 74.98) (width 0.2) (layer "F.Cu") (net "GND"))
 (segment (start 60.935 85.09) (end 61.5 85.655) (width 0.2) (layer "F.Cu") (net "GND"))
 (segment (start 78.8018 79.0762) (end 66.01 79.0762) (width 0.2) (layer "F.Cu") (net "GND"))
 (segment (start 65.7108 80.5272) (end 65.5012 80.3176) (width 0.2) (layer "F.Cu") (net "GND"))
 (segment (start 57.15 69.85) (end 57.15 69.4491) (width 0.2) (layer "F.Cu") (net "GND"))
 (segment (start 64.8912 85.3246) (end 64.8912 84.6667) (width 0.2) (layer "F.Cu") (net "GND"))
 (segment (start 58.8139 64.2022) (end 56.3483 66.6678) (width 0.2) (layer "F.Cu") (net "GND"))
 (segment (start 65.7108 80.5272) (end 65.7108 82.0137) (width 0.2) (layer "F.Cu") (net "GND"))
 (segment (start 57.15 69.4491) (end 57.15 69.0483) (width 0.2) (layer "F.Cu") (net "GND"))
 (segment (start 56.3483 66.6678) (end 56.3483 68.2466) (width 0.2) (layer "F.Cu") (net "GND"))
 (segment (start 65.7108 82.0137) (end 63.9745 83.75) (width 0.2) (layer "F.Cu") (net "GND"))
 (segment (start 64.5608 85.655) (end 64.8912 85.3246) (width 0.2) (layer "F.Cu") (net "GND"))
 (segment (start 80.7122 64.2022) (end 58.8139 64.2022) (width 0.2) (layer "F.Cu") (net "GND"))
 (segment (start 59.6774 69.4491) (end 65.2083 74.98) (width 0.2) (layer "F.Cu") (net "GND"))
 (segment (start 66.68 80.01) (end 66.68 80.5272) (width 0.2) (layer "F.Cu") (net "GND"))
 (segment (start 65.5012 80.3176) (end 65.5012 79.585) (width 0.2) (layer "F.Cu") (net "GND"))
 (segment (start 64.8912 84.6667) (end 63.9745 83.75) (width 0.2) (layer "F.Cu") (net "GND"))
 (segment (start 61.5 85.655) (end 64.5608 85.655) (width 0.2) (layer "F.Cu") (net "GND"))
 (segment (start 65.5012 79.585) (end 66.01 79.0762) (width 0.2) (layer "F.Cu") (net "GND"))
 (segment (start 63.9745 83.75) (end 63.56 83.75) (width 0.2) (layer "F.Cu") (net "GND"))
 (segment (start 68.51 74.98) (end 66.01 74.98) (width 0.2) (layer "F.Cu") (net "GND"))
 (segment (start 60.4579 84.5462) (end 63.0862 84.5462) (width 0.2) (layer "F.Cu") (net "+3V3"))
 (segment (start 60.295 84.7091) (end 60.4579 84.5462) (width 0.2) (layer "F.Cu") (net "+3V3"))
 (segment (start 57.4291 83.82) (end 58.1682 83.82) (width 0.2) (layer "F.Cu") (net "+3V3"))
 (segment (start 60.295 85.09) (end 60.295 84.7091) (width 0.2) (layer "F.Cu") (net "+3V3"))
 (segment (start 59.4059 83.82) (end 60.295 84.7091) (width 0.2) (layer "F.Cu") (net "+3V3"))
 (segment (start 57.4291 83.82) (end 59.4059 83.82) (width 0.2) (layer "F.Cu") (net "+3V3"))
 (segment (start 63.0862 84.5462) (end 63.56 85.02) (width 0.2) (layer "F.Cu") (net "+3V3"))
 (segment (start 58.1682 83.82) (end 57.4291 83.82) (width 0.2) (layer "F.Cu") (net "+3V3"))
 (via (at 57.4291 83.82) (size 0.6) (drill 0.3) (layers "F.Cu" "B.Cu") (capping no) (covering (front no) (back no))
  (plugging (front no) (back no)) (filling no) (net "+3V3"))
 (segment (start 57.15 72.39) (end 57.15 73.1917) (width 0.2) (layer "B.Cu") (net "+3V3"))
 (segment (start 57.15 73.1917) (end 57.9517 73.9934) (width 0.2) (layer "B.Cu") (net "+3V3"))
 (segment (start 57.9517 73.9934) (end 57.9517 83.2974) (width 0.2) (layer "B.Cu") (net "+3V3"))
 (segment (start 57.4291 83.82) (end 58.1682 83.82) (width 0.2) (layer "B.Cu") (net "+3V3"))
 (segment (start 57.9517 83.2974) (end 57.4291 83.82) (width 0.2) (layer "B.Cu") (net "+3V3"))
 (segment (start 58.1682 83.82) (end 57.4291 83.82) (width 0.2) (layer "B.Cu") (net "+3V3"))
 (segment (start 68.51 81.0298) (end 68.51 82.48) (width 0.2) (layer "F.Cu") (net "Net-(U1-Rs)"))
 (segment (start 66.04 79.786) (end 66.3481 79.4779) (width 0.2) (layer "F.Cu") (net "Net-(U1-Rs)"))
 (segment (start 66.3481 79.4779) (end 66.9581 79.4779) (width 0.2) (layer "F.Cu") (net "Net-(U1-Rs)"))
 (segment (start 66.9581 79.4779) (end 68.51 81.0298) (width 0.2) (layer "F.Cu") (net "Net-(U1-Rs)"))
 (segment (start 66.04 80.01) (end 66.04 79.786) (width 0.2) (layer "F.Cu") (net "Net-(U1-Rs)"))
 (segment (start 80.01 83.82) (end 80.7122 84.5222) (width 0.2) (layer "F.Cu") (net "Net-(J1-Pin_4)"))
 (segment (start 68.9431 83.3169) (end 72.4437 83.3169) (width 0.2) (layer "F.Cu") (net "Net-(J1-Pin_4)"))
 (segment (start 68.51 83.75) (end 68.9431 83.3169) (width 0.2) (layer "F.Cu") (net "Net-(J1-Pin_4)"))
 (segment (start 72.71 83.5832) (end 72.71 83.82) (width 0.2) (layer "F.Cu") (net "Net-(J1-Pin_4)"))
 (segment (start 72.4437 83.3169) (end 72.71 83.5832) (width 0.2) (layer "F.Cu") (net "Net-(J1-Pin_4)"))
 (segment (start 72.71 83.82) (end 80.01 83.82) (width 0.2) (layer "F.Cu") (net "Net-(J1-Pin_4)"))
 (segment (start 80.1791 62.8937) (end 79.3954 63.6774) (width 0.2) (layer "B.Cu") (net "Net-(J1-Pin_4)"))
 (segment (start 79.3954 63.6774) (end 79.3954 83.2054) (width 0.2) (layer "B.Cu") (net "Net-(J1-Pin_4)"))
 (segment (start 79.3954 83.2054) (end 80.7122 84.5222) (width 0.2) (layer "B.Cu") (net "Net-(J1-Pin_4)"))
 (segment (start 82.9393 62.8937) (end 80.1791 62.8937) (width 0.2) (layer "B.Cu") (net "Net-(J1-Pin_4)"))
 (segment (start 84.2478 64.2022) (end 82.9393 62.8937) (width 0.2) (layer "B.Cu") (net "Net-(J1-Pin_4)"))
 (segment (start 68.51 85.02) (end 68.9145 85.02) (width 0.2) (layer "F.Cu") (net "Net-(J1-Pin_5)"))
 (segment (start 71.665 87.7705) (end 71.665 91.44) (width 0.2) (layer "F.Cu") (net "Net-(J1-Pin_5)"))
 (segment (start 71.665 87.7705) (end 73.1455 86.29) (width 0.2) (layer "F.Cu") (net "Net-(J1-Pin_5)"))
 (segment (start 73.1455 86.29) (end 82.48 86.29) (width 0.2) (layer "F.Cu") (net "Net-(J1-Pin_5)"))
 (segment (start 68.9145 85.02) (end 71.665 87.7705) (width 0.2) (layer "F.Cu") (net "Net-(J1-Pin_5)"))
 (segment (start 82.48 65.97) (end 82.48 86.29) (width 0.2) (layer "B.Cu") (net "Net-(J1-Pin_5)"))
 (segment (start 62.5383 67.31) (end 70.2083 74.98) (width 0.2) (layer "F.Cu") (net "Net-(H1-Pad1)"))
 (segment (start 71.01 74.98) (end 70.2083 74.98) (width 0.2) (layer "F.Cu") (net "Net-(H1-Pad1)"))
 (segment (start 57.15 67.31) (end 62.5383 67.31) (width 0.2) (layer "F.Cu") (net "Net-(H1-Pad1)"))
 (segment (start 63.56 86.29) (end 59.1517 86.29) (width 0.2) (layer "F.Cu") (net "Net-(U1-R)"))
 (segment (start 57.15 85.09) (end 57.9517 85.09) (width 0.2) (layer "F.Cu") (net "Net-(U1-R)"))
 (segment (start 59.1517 86.29) (end 57.9517 85.09) (width 0.2) (layer "F.Cu") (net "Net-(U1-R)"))
 (segment (start 57.15 82.55) (end 57.9517 82.55) (width 0.2) (layer "F.Cu") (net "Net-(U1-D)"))
 (segment (start 63.56 82.48) (end 58.0217 82.48) (width 0.2) (layer "F.Cu") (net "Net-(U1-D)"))
 (segment (start 58.0217 82.48) (end 57.9517 82.55) (width 0.2) (layer "F.Cu") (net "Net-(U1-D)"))
 (segment (start 68.58 69.85) (end 79.5216 69.85) (width 0.2) (layer "F.Cu") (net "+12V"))
 (segment (start 84.4906 70.3505) (end 82.7995 68.6594) (width 0.2) (layer "F.Cu") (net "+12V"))
 (segment (start 80.7122 67.7378) (end 80.7122 68.6594) (width 0.2) (layer "F.Cu") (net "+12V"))
 (segment (start 79.5216 69.85) (end 80.7122 68.6594) (width 0.2) (layer "F.Cu") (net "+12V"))
 (segment (start 82.7995 68.6594) (end 80.7122 68.6594) (width 0.2) (layer "F.Cu") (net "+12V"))
 (via (at 68.58 69.85) (size 0.6) (drill 0.3) (layers "F.Cu" "B.Cu") (capping no) (covering (front no) (back no))
  (plugging (front no) (back no)) (filling no) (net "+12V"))
 (via (at 84.4906 70.3505) (size 0.6) (drill 0.3) (layers "F.Cu" "B.Cu") (capping no) (covering (front no) (back no))
  (plugging (front no) (back no)) (filling no) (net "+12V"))
 (segment (start 85.5721 71.432) (end 85.5721 86.7335) (width 0.2) (layer "B.Cu") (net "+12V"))
 (segment (start 85.5721 86.7335) (end 84.2478 88.0578) (width 0.2) (layer "B.Cu") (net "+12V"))
 (segment (start 63.51 71.5625) (end 63.51 74.98) (width 0.2) (layer "B.Cu") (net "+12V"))
 (segment (start 84.4906 70.3505) (end 85.5721 71.432) (width 0.2) (layer "B.Cu") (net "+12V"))
 (segment (start 68.58 69.85) (end 65.2225 69.85) (width 0.2) (layer "B.Cu") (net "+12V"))
 (segment (start 65.2225 69.85) (end 63.51 71.5625) (width 0.2) (layer "B.Cu") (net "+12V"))
 (segment (start 84.8118 89.3811) (end 85.9744 88.2185) (width 0.2) (layer "B.Cu") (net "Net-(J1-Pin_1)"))
 (segment (start 82.0355 89.3811) (end 84.8118 89.3811) (width 0.2) (layer "B.Cu") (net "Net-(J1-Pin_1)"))
 (segment (start 80.7122 88.0578) (end 82.0355 89.3811) (width 0.2) (layer "B.Cu") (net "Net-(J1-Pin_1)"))
 (segment (start 85.9744 88.2185) (end 85.9744 69.4644) (width 0.2) (layer "B.Cu") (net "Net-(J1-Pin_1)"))
 (segment (start 85.9744 69.4644) (end 84.2478 67.7378) (width 0.2) (layer "B.Cu") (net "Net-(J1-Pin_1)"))
 (segment (start 71.505 84.385) (end 72.07 83.82) (width 0.2) (layer "F.Cu") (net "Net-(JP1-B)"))
 (segment (start 67.2168 88.7103) (end 67.2168 84.6672) (width 0.2) (layer "F.Cu") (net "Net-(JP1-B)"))
 (segment (start 70.9982 92.4917) (end 67.2168 88.7103) (width 0.2) (layer "F.Cu") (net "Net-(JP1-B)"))
 (segment (start 67.499 84.385) (end 71.505 84.385) (width 0.2) (layer "F.Cu") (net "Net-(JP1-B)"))
 (segment (start 73.115 91.44) (end 73.115 92.4917) (width 0.2) (layer "F.Cu") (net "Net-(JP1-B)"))
 (segment (start 67.2168 84.6672) (end 67.499 84.385) (width 0.2) (layer "F.Cu") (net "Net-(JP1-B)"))
 (segment (start 73.115 92.4917) (end 70.9982 92.4917) (width 0.2) (layer "F.Cu") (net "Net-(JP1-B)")))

